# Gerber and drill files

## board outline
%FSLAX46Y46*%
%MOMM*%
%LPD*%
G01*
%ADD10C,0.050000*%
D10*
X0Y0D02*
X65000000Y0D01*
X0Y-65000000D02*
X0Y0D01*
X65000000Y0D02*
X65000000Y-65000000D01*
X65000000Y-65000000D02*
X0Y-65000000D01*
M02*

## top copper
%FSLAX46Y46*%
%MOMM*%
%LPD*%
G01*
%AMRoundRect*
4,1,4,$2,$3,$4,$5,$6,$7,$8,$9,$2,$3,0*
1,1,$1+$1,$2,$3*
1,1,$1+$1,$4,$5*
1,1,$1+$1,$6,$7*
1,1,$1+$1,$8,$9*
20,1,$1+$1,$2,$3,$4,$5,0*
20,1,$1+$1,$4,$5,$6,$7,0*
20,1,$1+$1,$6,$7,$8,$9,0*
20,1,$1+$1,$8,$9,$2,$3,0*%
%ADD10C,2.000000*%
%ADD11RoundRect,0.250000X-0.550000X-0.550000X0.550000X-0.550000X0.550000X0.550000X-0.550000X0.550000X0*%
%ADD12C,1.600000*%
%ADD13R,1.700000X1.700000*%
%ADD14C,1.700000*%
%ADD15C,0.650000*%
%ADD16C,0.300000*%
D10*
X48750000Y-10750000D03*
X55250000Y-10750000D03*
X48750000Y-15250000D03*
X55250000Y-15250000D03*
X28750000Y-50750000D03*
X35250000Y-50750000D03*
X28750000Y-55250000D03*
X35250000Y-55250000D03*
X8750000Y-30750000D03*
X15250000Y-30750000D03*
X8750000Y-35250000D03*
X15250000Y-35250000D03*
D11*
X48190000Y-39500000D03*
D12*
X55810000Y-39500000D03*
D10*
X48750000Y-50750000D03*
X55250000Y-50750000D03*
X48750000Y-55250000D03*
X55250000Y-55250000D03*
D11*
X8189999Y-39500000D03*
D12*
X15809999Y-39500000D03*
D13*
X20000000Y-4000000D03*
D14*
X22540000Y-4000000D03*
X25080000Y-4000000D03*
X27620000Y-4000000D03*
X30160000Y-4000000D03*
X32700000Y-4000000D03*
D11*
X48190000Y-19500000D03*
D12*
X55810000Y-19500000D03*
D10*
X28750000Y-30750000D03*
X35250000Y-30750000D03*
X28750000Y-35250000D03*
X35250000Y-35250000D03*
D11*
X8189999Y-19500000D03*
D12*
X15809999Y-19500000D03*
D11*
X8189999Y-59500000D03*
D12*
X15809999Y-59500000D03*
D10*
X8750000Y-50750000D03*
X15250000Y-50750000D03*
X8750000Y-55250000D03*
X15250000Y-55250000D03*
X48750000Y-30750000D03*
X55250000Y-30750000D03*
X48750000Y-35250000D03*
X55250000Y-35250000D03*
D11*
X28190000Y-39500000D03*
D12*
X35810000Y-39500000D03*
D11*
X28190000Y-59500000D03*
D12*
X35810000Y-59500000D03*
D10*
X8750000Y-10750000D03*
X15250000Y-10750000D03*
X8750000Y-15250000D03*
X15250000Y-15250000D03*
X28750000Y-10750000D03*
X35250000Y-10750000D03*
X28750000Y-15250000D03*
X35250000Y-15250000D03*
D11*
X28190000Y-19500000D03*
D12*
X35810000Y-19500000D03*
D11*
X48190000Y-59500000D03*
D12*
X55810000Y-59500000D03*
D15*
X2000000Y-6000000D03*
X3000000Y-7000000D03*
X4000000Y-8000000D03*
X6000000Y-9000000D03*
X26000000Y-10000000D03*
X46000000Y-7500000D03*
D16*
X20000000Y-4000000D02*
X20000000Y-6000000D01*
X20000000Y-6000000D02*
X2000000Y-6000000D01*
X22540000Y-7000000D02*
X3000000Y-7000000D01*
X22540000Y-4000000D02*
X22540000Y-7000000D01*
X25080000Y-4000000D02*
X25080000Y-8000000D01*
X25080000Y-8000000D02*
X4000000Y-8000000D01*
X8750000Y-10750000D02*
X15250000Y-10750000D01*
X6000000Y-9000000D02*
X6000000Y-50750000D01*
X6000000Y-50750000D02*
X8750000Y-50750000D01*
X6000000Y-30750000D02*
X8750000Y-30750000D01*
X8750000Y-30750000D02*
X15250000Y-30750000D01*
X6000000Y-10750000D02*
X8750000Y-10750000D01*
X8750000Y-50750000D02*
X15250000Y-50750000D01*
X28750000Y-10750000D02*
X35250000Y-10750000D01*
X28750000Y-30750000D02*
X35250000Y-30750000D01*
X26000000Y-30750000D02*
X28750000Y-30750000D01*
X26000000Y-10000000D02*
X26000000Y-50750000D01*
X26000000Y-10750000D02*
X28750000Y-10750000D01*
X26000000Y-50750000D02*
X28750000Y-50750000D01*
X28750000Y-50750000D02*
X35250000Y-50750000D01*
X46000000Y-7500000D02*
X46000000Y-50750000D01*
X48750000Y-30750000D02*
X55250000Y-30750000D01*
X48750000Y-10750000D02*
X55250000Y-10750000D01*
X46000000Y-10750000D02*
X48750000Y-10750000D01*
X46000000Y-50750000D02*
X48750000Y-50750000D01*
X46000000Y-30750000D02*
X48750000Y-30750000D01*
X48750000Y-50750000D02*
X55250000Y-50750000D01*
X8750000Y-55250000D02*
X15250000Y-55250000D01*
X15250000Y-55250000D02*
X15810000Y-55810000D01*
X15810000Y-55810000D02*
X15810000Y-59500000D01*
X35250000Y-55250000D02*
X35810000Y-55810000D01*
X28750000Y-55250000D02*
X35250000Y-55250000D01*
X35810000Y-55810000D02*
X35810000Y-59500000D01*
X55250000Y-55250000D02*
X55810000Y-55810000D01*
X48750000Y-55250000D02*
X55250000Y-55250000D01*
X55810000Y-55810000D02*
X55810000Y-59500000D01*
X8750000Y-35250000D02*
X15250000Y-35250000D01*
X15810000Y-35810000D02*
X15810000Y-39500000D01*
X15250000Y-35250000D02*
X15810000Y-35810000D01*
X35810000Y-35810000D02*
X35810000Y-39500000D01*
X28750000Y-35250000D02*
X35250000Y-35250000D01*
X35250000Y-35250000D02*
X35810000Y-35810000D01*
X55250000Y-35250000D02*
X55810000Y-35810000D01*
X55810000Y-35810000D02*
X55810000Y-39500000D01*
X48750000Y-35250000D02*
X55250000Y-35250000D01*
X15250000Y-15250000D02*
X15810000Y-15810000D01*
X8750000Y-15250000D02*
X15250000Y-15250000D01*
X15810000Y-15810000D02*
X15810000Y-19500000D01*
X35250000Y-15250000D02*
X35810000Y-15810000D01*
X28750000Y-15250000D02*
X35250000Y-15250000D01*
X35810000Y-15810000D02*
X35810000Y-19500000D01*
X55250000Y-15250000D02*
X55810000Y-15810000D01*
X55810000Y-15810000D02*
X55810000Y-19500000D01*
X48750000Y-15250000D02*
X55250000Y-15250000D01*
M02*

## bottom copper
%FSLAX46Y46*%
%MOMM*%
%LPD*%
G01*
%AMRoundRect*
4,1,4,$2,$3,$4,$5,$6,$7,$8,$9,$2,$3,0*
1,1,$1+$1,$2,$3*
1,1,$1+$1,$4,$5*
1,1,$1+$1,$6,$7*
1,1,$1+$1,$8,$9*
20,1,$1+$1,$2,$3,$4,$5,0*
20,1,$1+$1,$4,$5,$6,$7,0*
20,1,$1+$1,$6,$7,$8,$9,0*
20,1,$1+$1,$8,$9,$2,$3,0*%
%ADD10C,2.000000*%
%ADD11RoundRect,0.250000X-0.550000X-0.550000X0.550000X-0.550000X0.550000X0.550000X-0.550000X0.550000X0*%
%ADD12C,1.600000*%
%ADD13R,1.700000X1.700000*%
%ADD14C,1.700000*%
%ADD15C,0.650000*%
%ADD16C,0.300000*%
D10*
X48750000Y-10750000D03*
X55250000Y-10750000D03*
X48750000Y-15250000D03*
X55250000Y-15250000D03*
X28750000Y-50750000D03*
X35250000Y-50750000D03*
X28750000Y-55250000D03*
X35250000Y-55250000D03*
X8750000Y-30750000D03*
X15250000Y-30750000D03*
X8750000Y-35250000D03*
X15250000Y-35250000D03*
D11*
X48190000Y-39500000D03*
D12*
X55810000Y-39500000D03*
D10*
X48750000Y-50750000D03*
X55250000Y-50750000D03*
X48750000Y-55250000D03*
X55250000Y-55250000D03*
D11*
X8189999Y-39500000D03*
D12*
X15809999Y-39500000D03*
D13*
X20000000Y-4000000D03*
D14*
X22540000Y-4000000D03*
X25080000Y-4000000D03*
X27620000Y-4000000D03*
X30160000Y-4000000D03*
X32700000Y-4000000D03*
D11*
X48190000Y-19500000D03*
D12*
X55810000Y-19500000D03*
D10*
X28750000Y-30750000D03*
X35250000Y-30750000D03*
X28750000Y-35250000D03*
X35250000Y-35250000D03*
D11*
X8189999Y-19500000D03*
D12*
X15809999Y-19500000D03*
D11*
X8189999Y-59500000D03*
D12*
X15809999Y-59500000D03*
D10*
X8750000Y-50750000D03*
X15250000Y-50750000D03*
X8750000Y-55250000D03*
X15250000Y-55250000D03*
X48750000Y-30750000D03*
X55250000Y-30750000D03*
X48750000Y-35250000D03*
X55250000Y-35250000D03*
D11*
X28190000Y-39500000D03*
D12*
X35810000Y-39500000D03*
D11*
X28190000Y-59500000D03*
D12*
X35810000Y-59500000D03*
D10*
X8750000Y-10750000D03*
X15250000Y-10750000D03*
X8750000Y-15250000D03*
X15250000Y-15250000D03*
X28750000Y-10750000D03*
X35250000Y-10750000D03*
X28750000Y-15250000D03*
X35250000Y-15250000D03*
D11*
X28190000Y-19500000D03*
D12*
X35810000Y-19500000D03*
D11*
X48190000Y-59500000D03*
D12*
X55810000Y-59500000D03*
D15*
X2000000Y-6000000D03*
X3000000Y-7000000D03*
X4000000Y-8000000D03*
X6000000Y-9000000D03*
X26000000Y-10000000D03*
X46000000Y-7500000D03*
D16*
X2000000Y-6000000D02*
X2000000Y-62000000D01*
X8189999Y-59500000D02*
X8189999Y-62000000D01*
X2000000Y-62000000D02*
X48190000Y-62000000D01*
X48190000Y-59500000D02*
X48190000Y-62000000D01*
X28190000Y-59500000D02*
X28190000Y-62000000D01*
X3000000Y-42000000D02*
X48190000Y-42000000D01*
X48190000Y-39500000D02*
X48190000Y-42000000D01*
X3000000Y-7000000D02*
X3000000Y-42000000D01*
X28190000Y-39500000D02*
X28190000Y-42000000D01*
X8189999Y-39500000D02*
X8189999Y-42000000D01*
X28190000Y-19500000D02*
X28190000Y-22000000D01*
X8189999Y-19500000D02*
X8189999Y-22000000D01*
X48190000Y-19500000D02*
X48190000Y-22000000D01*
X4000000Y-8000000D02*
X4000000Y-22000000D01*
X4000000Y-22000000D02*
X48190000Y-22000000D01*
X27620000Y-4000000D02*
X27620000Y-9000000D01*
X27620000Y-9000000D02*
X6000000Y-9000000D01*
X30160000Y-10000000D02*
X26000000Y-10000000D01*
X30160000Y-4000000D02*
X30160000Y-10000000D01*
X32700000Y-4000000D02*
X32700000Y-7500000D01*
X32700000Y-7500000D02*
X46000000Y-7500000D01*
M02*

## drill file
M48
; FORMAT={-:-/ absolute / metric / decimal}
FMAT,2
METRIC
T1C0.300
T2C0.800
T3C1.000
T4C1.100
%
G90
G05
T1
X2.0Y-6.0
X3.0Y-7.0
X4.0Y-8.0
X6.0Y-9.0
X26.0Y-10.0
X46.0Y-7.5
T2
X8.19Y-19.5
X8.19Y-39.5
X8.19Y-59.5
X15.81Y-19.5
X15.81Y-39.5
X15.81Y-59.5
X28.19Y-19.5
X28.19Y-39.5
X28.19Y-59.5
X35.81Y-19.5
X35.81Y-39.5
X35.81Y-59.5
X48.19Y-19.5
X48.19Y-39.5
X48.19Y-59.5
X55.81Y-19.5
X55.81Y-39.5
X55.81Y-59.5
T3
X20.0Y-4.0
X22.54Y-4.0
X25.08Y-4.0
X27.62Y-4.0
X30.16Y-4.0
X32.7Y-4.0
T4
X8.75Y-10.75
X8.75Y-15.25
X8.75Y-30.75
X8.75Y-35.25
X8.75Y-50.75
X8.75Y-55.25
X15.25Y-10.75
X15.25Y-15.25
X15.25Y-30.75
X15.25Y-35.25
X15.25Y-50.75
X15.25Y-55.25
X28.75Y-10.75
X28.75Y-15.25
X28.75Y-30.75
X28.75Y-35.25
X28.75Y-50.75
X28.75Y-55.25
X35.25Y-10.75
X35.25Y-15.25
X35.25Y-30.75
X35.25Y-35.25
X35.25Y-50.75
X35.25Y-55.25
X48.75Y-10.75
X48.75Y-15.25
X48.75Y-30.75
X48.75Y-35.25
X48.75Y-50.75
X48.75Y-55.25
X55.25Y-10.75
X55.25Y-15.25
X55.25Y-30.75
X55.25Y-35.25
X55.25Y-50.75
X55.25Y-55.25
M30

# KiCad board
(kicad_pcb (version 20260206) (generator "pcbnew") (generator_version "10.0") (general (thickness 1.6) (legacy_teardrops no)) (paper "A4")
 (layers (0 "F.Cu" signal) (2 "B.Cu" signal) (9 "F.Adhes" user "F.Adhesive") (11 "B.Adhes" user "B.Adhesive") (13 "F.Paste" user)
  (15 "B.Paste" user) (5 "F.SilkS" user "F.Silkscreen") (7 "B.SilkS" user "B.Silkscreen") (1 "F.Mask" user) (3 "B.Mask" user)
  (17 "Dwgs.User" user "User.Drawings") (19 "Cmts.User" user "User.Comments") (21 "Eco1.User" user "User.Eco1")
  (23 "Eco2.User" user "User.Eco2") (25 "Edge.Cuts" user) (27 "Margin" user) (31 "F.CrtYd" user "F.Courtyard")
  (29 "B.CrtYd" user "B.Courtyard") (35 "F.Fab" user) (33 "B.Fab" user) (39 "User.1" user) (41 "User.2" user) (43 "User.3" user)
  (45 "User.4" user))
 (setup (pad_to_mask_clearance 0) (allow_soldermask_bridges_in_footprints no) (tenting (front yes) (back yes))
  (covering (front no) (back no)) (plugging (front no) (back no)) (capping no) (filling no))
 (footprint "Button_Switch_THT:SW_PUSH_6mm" (layer "F.Cu") (at 48.75 10.75)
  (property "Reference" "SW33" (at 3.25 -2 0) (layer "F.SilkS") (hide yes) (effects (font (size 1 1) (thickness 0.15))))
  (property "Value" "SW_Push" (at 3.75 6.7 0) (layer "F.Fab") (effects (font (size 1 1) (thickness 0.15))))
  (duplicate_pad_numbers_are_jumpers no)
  (pad "1" thru_hole circle (at 0 0 90) (size 2 2) (drill 1.1) (layers "*.Cu" "*.Mask") (remove_unused_layers no) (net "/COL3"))
  (pad "1" thru_hole circle (at 6.5 0 90) (size 2 2) (drill 1.1) (layers "*.Cu" "*.Mask") (remove_unused_layers no) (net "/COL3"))
  (pad "2" thru_hole circle (at 0 4.5 90) (size 2 2) (drill 1.1) (layers "*.Cu" "*.Mask") (remove_unused_layers no) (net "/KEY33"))
  (pad "2" thru_hole circle (at 6.5 4.5 90) (size 2 2) (drill 1.1) (layers "*.Cu" "*.Mask") (remove_unused_layers no) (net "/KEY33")))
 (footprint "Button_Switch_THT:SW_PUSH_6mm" (layer "F.Cu") (at 28.75 50.75)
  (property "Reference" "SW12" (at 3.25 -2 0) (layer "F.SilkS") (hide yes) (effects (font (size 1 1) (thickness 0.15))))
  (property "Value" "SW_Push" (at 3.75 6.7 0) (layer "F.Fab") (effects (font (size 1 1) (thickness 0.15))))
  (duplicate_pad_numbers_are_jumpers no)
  (pad "1" thru_hole circle (at 0 0 90) (size 2 2) (drill 1.1) (layers "*.Cu" "*.Mask") (remove_unused_layers no) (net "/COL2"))
  (pad "1" thru_hole circle (at 6.5 0 90) (size 2 2) (drill 1.1) (layers "*.Cu" "*.Mask") (remove_unused_layers no) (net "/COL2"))
  (pad "2" thru_hole circle (at 0 4.5 90) (size 2 2) (drill 1.1) (layers "*.Cu" "*.Mask") (remove_unused_layers no) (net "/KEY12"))
  (pad "2" thru_hole circle (at 6.5 4.5 90) (size 2 2) (drill 1.1) (layers "*.Cu" "*.Mask") (remove_unused_layers no) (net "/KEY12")))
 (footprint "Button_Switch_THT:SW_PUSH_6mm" (layer "F.Cu") (at 8.75 30.75)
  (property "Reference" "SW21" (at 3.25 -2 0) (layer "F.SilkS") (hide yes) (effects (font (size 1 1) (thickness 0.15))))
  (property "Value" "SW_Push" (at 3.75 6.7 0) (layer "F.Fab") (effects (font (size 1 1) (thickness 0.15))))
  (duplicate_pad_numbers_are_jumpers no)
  (pad "1" thru_hole circle (at 0 0 90) (size 2 2) (drill 1.1) (layers "*.Cu" "*.Mask") (remove_unused_layers no) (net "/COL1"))
  (pad "1" thru_hole circle (at 6.5 0 90) (size 2 2) (drill 1.1) (layers "*.Cu" "*.Mask") (remove_unused_layers no) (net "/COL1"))
  (pad "2" thru_hole circle (at 0 4.5 90) (size 2 2) (drill 1.1) (layers "*.Cu" "*.Mask") (remove_unused_layers no) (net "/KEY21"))
  (pad "2" thru_hole circle (at 6.5 4.5 90) (size 2 2) (drill 1.1) (layers "*.Cu" "*.Mask") (remove_unused_layers no) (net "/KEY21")))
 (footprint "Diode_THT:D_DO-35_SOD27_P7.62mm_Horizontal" (layer "F.Cu") (at 48.19 39.5)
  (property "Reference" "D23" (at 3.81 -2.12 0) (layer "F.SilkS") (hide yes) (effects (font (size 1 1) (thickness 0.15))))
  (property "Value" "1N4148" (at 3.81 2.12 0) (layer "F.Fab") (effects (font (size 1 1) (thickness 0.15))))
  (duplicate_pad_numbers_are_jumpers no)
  (pad "1" thru_hole roundrect (at 0 0) (size 1.6 1.6) (drill 0.8) (layers "*.Cu" "*.Mask") (remove_unused_layers no)
   (roundrect_rratio 0.15625) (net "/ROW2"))
  (pad "2" thru_hole circle (at 7.62 0) (size 1.6 1.6) (drill 0.8) (layers "*.Cu" "*.Mask") (remove_unused_layers no) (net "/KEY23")))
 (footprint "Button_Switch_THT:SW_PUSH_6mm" (layer "F.Cu") (at 48.75 50.75)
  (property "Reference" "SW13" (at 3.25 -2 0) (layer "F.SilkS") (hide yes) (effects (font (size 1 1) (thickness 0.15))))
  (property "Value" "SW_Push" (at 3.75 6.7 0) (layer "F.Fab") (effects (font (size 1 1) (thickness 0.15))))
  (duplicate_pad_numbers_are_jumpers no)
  (pad "1" thru_hole circle (at 0 0 90) (size 2 2) (drill 1.1) (layers "*.Cu" "*.Mask") (remove_unused_layers no) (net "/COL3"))
  (pad "1" thru_hole circle (at 6.5 0 90) (size 2 2) (drill 1.1) (layers "*.Cu" "*.Mask") (remove_unused_layers no) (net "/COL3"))
  (pad "2" thru_hole circle (at 0 4.5 90) (size 2 2) (drill 1.1) (layers "*.Cu" "*.Mask") (remove_unused_layers no) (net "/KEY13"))
  (pad "2" thru_hole circle (at 6.5 4.5 90) (size 2 2) (drill 1.1) (layers "*.Cu" "*.Mask") (remove_unused_layers no) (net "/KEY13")))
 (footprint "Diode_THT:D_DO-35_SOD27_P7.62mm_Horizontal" (layer "F.Cu") (at 8.189999 39.5)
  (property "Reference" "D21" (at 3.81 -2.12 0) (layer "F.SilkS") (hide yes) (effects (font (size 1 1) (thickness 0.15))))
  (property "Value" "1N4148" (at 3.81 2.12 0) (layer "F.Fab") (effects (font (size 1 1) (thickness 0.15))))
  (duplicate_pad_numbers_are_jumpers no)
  (pad "1" thru_hole roundrect (at 0 0) (size 1.6 1.6) (drill 0.8) (layers "*.Cu" "*.Mask") (remove_unused_layers no)
   (roundrect_rratio 0.15625) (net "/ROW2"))
  (pad "2" thru_hole circle (at 7.62 0) (size 1.6 1.6) (drill 0.8) (layers "*.Cu" "*.Mask") (remove_unused_layers no) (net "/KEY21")))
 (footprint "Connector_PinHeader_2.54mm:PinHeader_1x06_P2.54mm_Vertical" (layer "F.Cu") (at 20 4 90)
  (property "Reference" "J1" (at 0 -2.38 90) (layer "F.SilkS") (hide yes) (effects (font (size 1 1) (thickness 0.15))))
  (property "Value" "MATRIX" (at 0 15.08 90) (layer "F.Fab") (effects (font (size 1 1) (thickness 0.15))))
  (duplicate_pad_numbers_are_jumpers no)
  (pad "1" thru_hole rect (at 0 0 90) (size 1.7 1.7) (drill 1) (layers "*.Cu" "*.Mask") (remove_unused_layers no) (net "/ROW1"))
  (pad "2" thru_hole circle (at 0 2.54 90) (size 1.7 1.7) (drill 1) (layers "*.Cu" "*.Mask") (remove_unused_layers no) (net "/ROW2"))
  (pad "3" thru_hole circle (at 0 5.08 90) (size 1.7 1.7) (drill 1) (layers "*.Cu" "*.Mask") (remove_unused_layers no) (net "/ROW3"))
  (pad "4" thru_hole circle (at 0 7.62 90) (size 1.7 1.7) (drill 1) (layers "*.Cu" "*.Mask") (remove_unused_layers no) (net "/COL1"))
  (pad "5" thru_hole circle (at 0 10.16 90) (size 1.7 1.7) (drill 1) (layers "*.Cu" "*.Mask") (remove_unused_layers no) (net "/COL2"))
  (pad "6" thru_hole circle (at 0 12.7 90) (size 1.7 1.7) (drill 1) (layers "*.Cu" "*.Mask") (remove_unused_layers no) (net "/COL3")))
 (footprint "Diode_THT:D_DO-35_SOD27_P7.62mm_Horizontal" (layer "F.Cu") (at 48.19 19.5)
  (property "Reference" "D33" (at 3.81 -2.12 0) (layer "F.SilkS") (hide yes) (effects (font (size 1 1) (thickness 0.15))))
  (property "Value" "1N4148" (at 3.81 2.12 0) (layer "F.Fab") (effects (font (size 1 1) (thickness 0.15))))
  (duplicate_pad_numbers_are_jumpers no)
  (pad "1" thru_hole roundrect (at 0 0) (size 1.6 1.6) (drill 0.8) (layers "*.Cu" "*.Mask") (remove_unused_layers no)
   (roundrect_rratio 0.15625) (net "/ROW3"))
  (pad "2" thru_hole circle (at 7.62 0) (size 1.6 1.6) (drill 0.8) (layers "*.Cu" "*.Mask") (remove_unused_layers no) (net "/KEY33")))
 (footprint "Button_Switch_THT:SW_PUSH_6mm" (layer "F.Cu") (at 28.75 30.75)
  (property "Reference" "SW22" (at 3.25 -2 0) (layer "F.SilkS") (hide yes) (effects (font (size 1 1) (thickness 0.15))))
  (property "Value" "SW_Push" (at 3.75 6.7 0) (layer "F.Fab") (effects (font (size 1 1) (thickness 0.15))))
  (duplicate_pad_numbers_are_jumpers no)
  (pad "1" thru_hole circle (at 0 0 90) (size 2 2) (drill 1.1) (layers "*.Cu" "*.Mask") (remove_unused_layers no) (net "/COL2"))
  (pad "1" thru_hole circle (at 6.5 0 90) (size 2 2) (drill 1.1) (layers "*.Cu" "*.Mask") (remove_unused_layers no) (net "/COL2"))
  (pad "2" thru_hole circle (at 0 4.5 90) (size 2 2) (drill 1.1) (layers "*.Cu" "*.Mask") (remove_unused_layers no) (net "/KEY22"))
  (pad "2" thru_hole circle (at 6.5 4.5 90) (size 2 2) (drill 1.1) (layers "*.Cu" "*.Mask") (remove_unused_layers no) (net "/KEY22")))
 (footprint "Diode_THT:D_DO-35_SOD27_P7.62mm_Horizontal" (layer "F.Cu") (at 8.189999 19.5)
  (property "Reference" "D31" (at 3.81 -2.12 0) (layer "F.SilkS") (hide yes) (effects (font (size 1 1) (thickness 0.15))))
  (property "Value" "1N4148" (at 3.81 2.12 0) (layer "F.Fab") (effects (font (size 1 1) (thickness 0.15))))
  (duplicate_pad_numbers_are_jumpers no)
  (pad "1" thru_hole roundrect (at 0 0) (size 1.6 1.6) (drill 0.8) (layers "*.Cu" "*.Mask") (remove_unused_layers no)
   (roundrect_rratio 0.15625) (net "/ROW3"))
  (pad "2" thru_hole circle (at 7.62 0) (size 1.6 1.6) (drill 0.8) (layers "*.Cu" "*.Mask") (remove_unused_layers no) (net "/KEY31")))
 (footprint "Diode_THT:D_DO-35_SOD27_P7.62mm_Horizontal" (layer "F.Cu") (at 8.189999 59.5)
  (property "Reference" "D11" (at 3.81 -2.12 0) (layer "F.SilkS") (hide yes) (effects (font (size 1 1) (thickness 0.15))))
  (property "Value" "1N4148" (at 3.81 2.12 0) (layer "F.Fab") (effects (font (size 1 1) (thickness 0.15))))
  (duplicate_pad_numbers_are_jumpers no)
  (pad "1" thru_hole roundrect (at 0 0) (size 1.6 1.6) (drill 0.8) (layers "*.Cu" "*.Mask") (remove_unused_layers no)
   (roundrect_rratio 0.15625) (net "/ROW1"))
  (pad "2" thru_hole circle (at 7.62 0) (size 1.6 1.6) (drill 0.8) (layers "*.Cu" "*.Mask") (remove_unused_layers no) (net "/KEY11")))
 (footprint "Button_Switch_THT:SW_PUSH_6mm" (layer "F.Cu") (at 8.75 50.75)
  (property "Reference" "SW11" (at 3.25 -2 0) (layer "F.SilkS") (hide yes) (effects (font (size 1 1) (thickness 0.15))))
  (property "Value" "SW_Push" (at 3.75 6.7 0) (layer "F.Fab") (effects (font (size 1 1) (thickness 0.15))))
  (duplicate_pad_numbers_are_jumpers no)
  (pad "1" thru_hole circle (at 0 0 90) (size 2 2) (drill 1.1) (layers "*.Cu" "*.Mask") (remove_unused_layers no) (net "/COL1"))
  (pad "1" thru_hole circle (at 6.5 0 90) (size 2 2) (drill 1.1) (layers "*.Cu" "*.Mask") (remove_unused_layers no) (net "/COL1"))
  (pad "2" thru_hole circle (at 0 4.5 90) (size 2 2) (drill 1.1) (layers "*.Cu" "*.Mask") (remove_unused_layers no) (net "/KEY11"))
  (pad "2" thru_hole circle (at 6.5 4.5 90) (size 2 2) (drill 1.1) (layers "*.Cu" "*.Mask") (remove_unused_layers no) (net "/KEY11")))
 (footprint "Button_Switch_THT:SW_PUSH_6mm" (layer "F.Cu") (at 48.75 30.75)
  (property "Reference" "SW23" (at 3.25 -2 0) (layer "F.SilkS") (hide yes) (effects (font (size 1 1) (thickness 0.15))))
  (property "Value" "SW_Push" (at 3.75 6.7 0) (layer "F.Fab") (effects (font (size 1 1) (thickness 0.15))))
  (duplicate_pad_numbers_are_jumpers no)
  (pad "1" thru_hole circle (at 0 0 90) (size 2 2) (drill 1.1) (layers "*.Cu" "*.Mask") (remove_unused_layers no) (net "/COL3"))
  (pad "1" thru_hole circle (at 6.5 0 90) (size 2 2) (drill 1.1) (layers "*.Cu" "*.Mask") (remove_unused_layers no) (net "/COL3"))
  (pad "2" thru_hole circle (at 0 4.5 90) (size 2 2) (drill 1.1) (layers "*.Cu" "*.Mask") (remove_unused_layers no) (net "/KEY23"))
  (pad "2" thru_hole circle (at 6.5 4.5 90) (size 2 2) (drill 1.1) (layers "*.Cu" "*.Mask") (remove_unused_layers no) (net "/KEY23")))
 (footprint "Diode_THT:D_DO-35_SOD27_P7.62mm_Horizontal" (layer "F.Cu") (at 28.19 39.5)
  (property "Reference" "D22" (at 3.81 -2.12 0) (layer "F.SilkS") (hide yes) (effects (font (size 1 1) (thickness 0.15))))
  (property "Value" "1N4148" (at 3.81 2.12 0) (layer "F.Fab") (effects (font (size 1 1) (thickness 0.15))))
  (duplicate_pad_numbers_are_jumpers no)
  (pad "1" thru_hole roundrect (at 0 0) (size 1.6 1.6) (drill 0.8) (layers "*.Cu" "*.Mask") (remove_unused_layers no)
   (roundrect_rratio 0.15625) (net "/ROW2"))
  (pad "2" thru_hole circle (at 7.62 0) (size 1.6 1.6) (drill 0.8) (layers "*.Cu" "*.Mask") (remove_unused_layers no) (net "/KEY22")))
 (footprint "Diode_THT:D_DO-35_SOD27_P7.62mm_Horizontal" (layer "F.Cu") (at 28.19 59.5)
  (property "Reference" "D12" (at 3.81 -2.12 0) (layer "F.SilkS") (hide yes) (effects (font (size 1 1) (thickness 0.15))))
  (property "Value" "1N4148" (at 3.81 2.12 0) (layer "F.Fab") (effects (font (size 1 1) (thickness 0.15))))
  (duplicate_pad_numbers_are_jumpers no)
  (pad "1" thru_hole roundrect (at 0 0) (size 1.6 1.6) (drill 0.8) (layers "*.Cu" "*.Mask") (remove_unused_layers no)
   (roundrect_rratio 0.15625) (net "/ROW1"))
  (pad "2" thru_hole circle (at 7.62 0) (size 1.6 1.6) (drill 0.8) (layers "*.Cu" "*.Mask") (remove_unused_layers no) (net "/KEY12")))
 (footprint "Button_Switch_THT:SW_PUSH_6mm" (layer "F.Cu") (at 8.75 10.75)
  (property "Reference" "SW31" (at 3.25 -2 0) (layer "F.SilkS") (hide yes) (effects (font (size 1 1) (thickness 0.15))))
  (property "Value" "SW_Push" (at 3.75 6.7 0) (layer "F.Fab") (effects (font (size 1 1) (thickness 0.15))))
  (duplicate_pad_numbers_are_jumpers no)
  (pad "1" thru_hole circle (at 0 0 90) (size 2 2) (drill 1.1) (layers "*.Cu" "*.Mask") (remove_unused_layers no) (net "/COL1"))
  (pad "1" thru_hole circle (at 6.5 0 90) (size 2 2) (drill 1.1) (layers "*.Cu" "*.Mask") (remove_unused_layers no) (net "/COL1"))
  (pad "2" thru_hole circle (at 0 4.5 90) (size 2 2) (drill 1.1) (layers "*.Cu" "*.Mask") (remove_unused_layers no) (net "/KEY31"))
  (pad "2" thru_hole circle (at 6.5 4.5 90) (size 2 2) (drill 1.1) (layers "*.Cu" "*.Mask") (remove_unused_layers no) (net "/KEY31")))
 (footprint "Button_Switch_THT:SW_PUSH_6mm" (layer "F.Cu") (at 28.75 10.75)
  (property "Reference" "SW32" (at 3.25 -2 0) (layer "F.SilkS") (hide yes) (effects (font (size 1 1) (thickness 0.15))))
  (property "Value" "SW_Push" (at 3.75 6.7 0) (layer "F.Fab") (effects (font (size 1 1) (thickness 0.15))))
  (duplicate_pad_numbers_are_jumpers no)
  (pad "1" thru_hole circle (at 0 0 90) (size 2 2) (drill 1.1) (layers "*.Cu" "*.Mask") (remove_unused_layers no) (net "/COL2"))
  (pad "1" thru_hole circle (at 6.5 0 90) (size 2 2) (drill 1.1) (layers "*.Cu" "*.Mask") (remove_unused_layers no) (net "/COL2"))
  (pad "2" thru_hole circle (at 0 4.5 90) (size 2 2) (drill 1.1) (layers "*.Cu" "*.Mask") (remove_unused_layers no) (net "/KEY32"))
  (pad "2" thru_hole circle (at 6.5 4.5 90) (size 2 2) (drill 1.1) (layers "*.Cu" "*.Mask") (remove_unused_layers no) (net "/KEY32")))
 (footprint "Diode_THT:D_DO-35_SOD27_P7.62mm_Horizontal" (layer "F.Cu") (at 28.19 19.5)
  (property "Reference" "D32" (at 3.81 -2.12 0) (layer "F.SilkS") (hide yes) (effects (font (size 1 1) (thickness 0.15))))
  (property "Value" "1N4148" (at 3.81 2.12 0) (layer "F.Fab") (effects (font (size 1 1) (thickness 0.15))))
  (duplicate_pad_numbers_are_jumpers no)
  (pad "1" thru_hole roundrect (at 0 0) (size 1.6 1.6) (drill 0.8) (layers "*.Cu" "*.Mask") (remove_unused_layers no)
   (roundrect_rratio 0.15625) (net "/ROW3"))
  (pad "2" thru_hole circle (at 7.62 0) (size 1.6 1.6) (drill 0.8) (layers "*.Cu" "*.Mask") (remove_unused_layers no) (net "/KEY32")))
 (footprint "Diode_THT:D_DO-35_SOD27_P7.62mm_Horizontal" (layer "F.Cu") (at 48.19 59.5)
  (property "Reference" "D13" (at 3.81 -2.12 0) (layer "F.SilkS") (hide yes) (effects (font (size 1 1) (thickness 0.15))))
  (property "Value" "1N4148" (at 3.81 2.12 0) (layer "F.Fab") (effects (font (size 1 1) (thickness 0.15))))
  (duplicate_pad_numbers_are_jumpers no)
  (pad "1" thru_hole roundrect (at 0 0) (size 1.6 1.6) (drill 0.8) (layers "*.Cu" "*.Mask") (remove_unused_layers no)
   (roundrect_rratio 0.15625) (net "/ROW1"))
  (pad "2" thru_hole circle (at 7.62 0) (size 1.6 1.6) (drill 0.8) (layers "*.Cu" "*.Mask") (remove_unused_layers no) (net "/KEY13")))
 (gr_line (start 0 0) (end 65 0) (stroke (width 0.05) (type default)) (layer "Edge.Cuts"))
 (gr_line (start 0 65) (end 0 0) (stroke (width 0.05) (type default)) (layer "Edge.Cuts"))
 (gr_line (start 65 0) (end 65 65) (stroke (width 0.05) (type default)) (layer "Edge.Cuts"))
 (gr_line (start 65 65) (end 0 65) (stroke (width 0.05) (type default)) (layer "Edge.Cuts"))
 (segment (start 20 4) (end 20 6) (width 0.3) (layer "F.Cu") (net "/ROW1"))
 (segment (start 20 6) (end 2 6) (width 0.3) (layer "F.Cu") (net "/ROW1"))
 (via (at 2 6) (size 0.65) (drill 0.3) (layers "F.Cu" "B.Cu") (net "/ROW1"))
 (segment (start 2 6) (end 2 62) (width 0.3) (layer "B.Cu") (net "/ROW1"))
 (segment (start 8.189999 59.5) (end 8.189999 62) (width 0.3) (layer "B.Cu") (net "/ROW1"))
 (segment (start 2 62) (end 48.19 62) (width 0.3) (layer "B.Cu") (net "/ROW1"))
 (segment (start 48.19 59.5) (end 48.19 62) (width 0.3) (layer "B.Cu") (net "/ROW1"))
 (segment (start 28.19 59.5) (end 28.19 62) (width 0.3) (layer "B.Cu") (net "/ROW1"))
 (segment (start 22.54 7) (end 3 7) (width 0.3) (layer "F.Cu") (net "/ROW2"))
 (segment (start 22.54 4) (end 22.54 7) (width 0.3) (layer "F.Cu") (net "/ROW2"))
 (via (at 3 7) (size 0.65) (drill 0.3) (layers "F.Cu" "B.Cu") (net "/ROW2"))
 (segment (start 3 42) (end 48.19 42) (width 0.3) (layer "B.Cu") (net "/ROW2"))
 (segment (start 48.19 39.5) (end 48.19 42) (width 0.3) (layer "B.Cu") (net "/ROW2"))
 (segment (start 3 7) (end 3 42) (width 0.3) (layer "B.Cu") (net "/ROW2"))
 (segment (start 28.19 39.5) (end 28.19 42) (width 0.3) (layer "B.Cu") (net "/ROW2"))
 (segment (start 8.189999 39.5) (end 8.189999 42) (width 0.3) (layer "B.Cu") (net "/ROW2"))
 (segment (start 25.08 4) (end 25.08 8) (width 0.3) (layer "F.Cu") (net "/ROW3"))
 (segment (start 25.08 8) (end 4 8) (width 0.3) (layer "F.Cu") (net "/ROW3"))
 (via (at 4 8) (size 0.65) (drill 0.3) (layers "F.Cu" "B.Cu") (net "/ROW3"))
 (segment (start 28.19 19.5) (end 28.19 22) (width 0.3) (layer "B.Cu") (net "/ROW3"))
 (segment (start 8.189999 19.5) (end 8.189999 22) (width 0.3) (layer "B.Cu") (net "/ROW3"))
 (segment (start 48.19 19.5) (end 48.19 22) (width 0.3) (layer "B.Cu") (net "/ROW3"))
 (segment (start 4 8) (end 4 22) (width 0.3) (layer "B.Cu") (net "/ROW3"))
 (segment (start 4 22) (end 48.19 22) (width 0.3) (layer "B.Cu") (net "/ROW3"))
 (segment (start 8.75 10.75) (end 15.25 10.75) (width 0.3) (layer "F.Cu") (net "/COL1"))
 (segment (start 6 9) (end 6 50.75) (width 0.3) (layer "F.Cu") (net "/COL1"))
 (segment (start 6 50.75) (end 8.75 50.75) (width 0.3) (layer "F.Cu") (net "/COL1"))
 (segment (start 6 30.75) (end 8.75 30.75) (width 0.3) (layer "F.Cu") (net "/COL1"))
 (segment (start 8.75 30.75) (end 15.25 30.75) (width 0.3) (layer "F.Cu") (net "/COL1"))
 (segment (start 6 10.75) (end 8.75 10.75) (width 0.3) (layer "F.Cu") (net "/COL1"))
 (segment (start 8.75 50.75) (end 15.25 50.75) (width 0.3) (layer "F.Cu") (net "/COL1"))
 (via (at 6 9) (size 0.65) (drill 0.3) (layers "F.Cu" "B.Cu") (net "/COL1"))
 (segment (start 27.62 4) (end 27.62 9) (width 0.3) (layer "B.Cu") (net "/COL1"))
 (segment (start 27.62 9) (end 6 9) (width 0.3) (layer "B.Cu") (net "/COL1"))
 (segment (start 28.75 10.75) (end 35.25 10.75) (width 0.3) (layer "F.Cu") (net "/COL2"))
 (segment (start 28.75 30.75) (end 35.25 30.75) (width 0.3) (layer "F.Cu") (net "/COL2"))
 (segment (start 26 30.75) (end 28.75 30.75) (width 0.3) (layer "F.Cu") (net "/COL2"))
 (segment (start 26 10) (end 26 50.75) (width 0.3) (layer "F.Cu") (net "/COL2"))
 (segment (start 26 10.75) (end 28.75 10.75) (width 0.3) (layer "F.Cu") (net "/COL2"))
 (segment (start 26 50.75) (end 28.75 50.75) (width 0.3) (layer "F.Cu") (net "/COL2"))
 (segment (start 28.75 50.75) (end 35.25 50.75) (width 0.3) (layer "F.Cu") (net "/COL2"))
 (via (at 26 10) (size 0.65) (drill 0.3) (layers "F.Cu" "B.Cu") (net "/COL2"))
 (segment (start 30.16 10) (end 26 10) (width 0.3) (layer "B.Cu") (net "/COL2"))
 (segment (start 30.16 4) (end 30.16 10) (width 0.3) (layer "B.Cu") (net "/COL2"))
 (segment (start 46 7.5) (end 46 50.75) (width 0.3) (layer "F.Cu") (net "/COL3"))
 (segment (start 48.75 30.75) (end 55.25 30.75) (width 0.3) (layer "F.Cu") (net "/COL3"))
 (segment (start 48.75 10.75) (end 55.25 10.75) (width 0.3) (layer "F.Cu") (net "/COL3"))
 (segment (start 46 10.75) (end 48.75 10.75) (width 0.3) (layer "F.Cu") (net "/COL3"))
 (segment (start 46 50.75) (end 48.75 50.75) (width 0.3) (layer "F.Cu") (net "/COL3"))
 (segment (start 46 30.75) (end 48.75 30.75) (width 0.3) (layer "F.Cu") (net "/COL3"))
 (segment (start 48.75 50.75) (end 55.25 50.75) (width 0.3) (layer "F.Cu") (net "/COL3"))
 (via (at 46 7.5) (size 0.65) (drill 0.3) (layers "F.Cu" "B.Cu") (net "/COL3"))
 (segment (start 32.7 4) (end 32.7 7.5) (width 0.3) (layer "B.Cu") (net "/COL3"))
 (segment (start 32.7 7.5) (end 46 7.5) (width 0.3) (layer "B.Cu") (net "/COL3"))
 (segment (start 8.75 55.25) (end 15.25 55.25) (width 0.3) (layer "F.Cu") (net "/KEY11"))
 (segment (start 15.25 55.25) (end 15.81 55.81) (width 0.3) (layer "F.Cu") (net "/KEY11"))
 (segment (start 15.81 55.81) (end 15.81 59.5) (width 0.3) (layer "F.Cu") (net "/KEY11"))
 (segment (start 35.25 55.25) (end 35.81 55.81) (width 0.3) (layer "F.Cu") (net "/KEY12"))
 (segment (start 28.75 55.25) (end 35.25 55.25) (width 0.3) (layer "F.Cu") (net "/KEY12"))
 (segment (start 35.81 55.81) (end 35.81 59.5) (width 0.3) (layer "F.Cu") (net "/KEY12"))
 (segment (start 55.25 55.25) (end 55.81 55.81) (width 0.3) (layer "F.Cu") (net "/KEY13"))
 (segment (start 48.75 55.25) (end 55.25 55.25) (width 0.3) (layer "F.Cu") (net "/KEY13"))
 (segment (start 55.81 55.81) (end 55.81 59.5) (width 0.3) (layer "F.Cu") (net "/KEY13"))
 (segment (start 8.75 35.25) (end 15.25 35.25) (width 0.3) (layer "F.Cu") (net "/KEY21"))
 (segment (start 15.81 35.81) (end 15.81 39.5) (width 0.3) (layer "F.Cu") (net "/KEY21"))
 (segment (start 15.25 35.25) (end 15.81 35.81) (width 0.3) (layer "F.Cu") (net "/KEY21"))
 (segment (start 35.81 35.81) (end 35.81 39.5) (width 0.3) (layer "F.Cu") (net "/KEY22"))
 (segment (start 28.75 35.25) (end 35.25 35.25) (width 0.3) (layer "F.Cu") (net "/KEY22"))
 (segment (start 35.25 35.25) (end 35.81 35.81) (width 0.3) (layer "F.Cu") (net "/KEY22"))
 (segment (start 55.25 35.25) (end 55.81 35.81) (width 0.3) (layer "F.Cu") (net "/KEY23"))
 (segment (start 55.81 35.81) (end 55.81 39.5) (width 0.3) (layer "F.Cu") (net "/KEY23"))
 (segment (start 48.75 35.25) (end 55.25 35.25) (width 0.3) (layer "F.Cu") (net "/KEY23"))
 (segment (start 15.25 15.25) (end 15.81 15.81) (width 0.3) (layer "F.Cu") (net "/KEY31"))
 (segment (start 8.75 15.25) (end 15.25 15.25) (width 0.3) (layer "F.Cu") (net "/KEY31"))
 (segment (start 15.81 15.81) (end 15.81 19.5) (width 0.3) (layer "F.Cu") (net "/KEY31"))
 (segment (start 35.25 15.25) (end 35.81 15.81) (width 0.3) (layer "F.Cu") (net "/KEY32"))
 (segment (start 28.75 15.25) (end 35.25 15.25) (width 0.3) (layer "F.Cu") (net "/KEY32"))
 (segment (start 35.81 15.81) (end 35.81 19.5) (width 0.3) (layer "F.Cu") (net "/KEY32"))
 (segment (start 55.25 15.25) (end 55.81 15.81) (width 0.3) (layer "F.Cu") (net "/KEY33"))
 (segment (start 55.81 15.81) (end 55.81 19.5) (width 0.3) (layer "F.Cu") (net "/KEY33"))
 (segment (start 48.75 15.25) (end 55.25 15.25) (width 0.3) (layer "F.Cu") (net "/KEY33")))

